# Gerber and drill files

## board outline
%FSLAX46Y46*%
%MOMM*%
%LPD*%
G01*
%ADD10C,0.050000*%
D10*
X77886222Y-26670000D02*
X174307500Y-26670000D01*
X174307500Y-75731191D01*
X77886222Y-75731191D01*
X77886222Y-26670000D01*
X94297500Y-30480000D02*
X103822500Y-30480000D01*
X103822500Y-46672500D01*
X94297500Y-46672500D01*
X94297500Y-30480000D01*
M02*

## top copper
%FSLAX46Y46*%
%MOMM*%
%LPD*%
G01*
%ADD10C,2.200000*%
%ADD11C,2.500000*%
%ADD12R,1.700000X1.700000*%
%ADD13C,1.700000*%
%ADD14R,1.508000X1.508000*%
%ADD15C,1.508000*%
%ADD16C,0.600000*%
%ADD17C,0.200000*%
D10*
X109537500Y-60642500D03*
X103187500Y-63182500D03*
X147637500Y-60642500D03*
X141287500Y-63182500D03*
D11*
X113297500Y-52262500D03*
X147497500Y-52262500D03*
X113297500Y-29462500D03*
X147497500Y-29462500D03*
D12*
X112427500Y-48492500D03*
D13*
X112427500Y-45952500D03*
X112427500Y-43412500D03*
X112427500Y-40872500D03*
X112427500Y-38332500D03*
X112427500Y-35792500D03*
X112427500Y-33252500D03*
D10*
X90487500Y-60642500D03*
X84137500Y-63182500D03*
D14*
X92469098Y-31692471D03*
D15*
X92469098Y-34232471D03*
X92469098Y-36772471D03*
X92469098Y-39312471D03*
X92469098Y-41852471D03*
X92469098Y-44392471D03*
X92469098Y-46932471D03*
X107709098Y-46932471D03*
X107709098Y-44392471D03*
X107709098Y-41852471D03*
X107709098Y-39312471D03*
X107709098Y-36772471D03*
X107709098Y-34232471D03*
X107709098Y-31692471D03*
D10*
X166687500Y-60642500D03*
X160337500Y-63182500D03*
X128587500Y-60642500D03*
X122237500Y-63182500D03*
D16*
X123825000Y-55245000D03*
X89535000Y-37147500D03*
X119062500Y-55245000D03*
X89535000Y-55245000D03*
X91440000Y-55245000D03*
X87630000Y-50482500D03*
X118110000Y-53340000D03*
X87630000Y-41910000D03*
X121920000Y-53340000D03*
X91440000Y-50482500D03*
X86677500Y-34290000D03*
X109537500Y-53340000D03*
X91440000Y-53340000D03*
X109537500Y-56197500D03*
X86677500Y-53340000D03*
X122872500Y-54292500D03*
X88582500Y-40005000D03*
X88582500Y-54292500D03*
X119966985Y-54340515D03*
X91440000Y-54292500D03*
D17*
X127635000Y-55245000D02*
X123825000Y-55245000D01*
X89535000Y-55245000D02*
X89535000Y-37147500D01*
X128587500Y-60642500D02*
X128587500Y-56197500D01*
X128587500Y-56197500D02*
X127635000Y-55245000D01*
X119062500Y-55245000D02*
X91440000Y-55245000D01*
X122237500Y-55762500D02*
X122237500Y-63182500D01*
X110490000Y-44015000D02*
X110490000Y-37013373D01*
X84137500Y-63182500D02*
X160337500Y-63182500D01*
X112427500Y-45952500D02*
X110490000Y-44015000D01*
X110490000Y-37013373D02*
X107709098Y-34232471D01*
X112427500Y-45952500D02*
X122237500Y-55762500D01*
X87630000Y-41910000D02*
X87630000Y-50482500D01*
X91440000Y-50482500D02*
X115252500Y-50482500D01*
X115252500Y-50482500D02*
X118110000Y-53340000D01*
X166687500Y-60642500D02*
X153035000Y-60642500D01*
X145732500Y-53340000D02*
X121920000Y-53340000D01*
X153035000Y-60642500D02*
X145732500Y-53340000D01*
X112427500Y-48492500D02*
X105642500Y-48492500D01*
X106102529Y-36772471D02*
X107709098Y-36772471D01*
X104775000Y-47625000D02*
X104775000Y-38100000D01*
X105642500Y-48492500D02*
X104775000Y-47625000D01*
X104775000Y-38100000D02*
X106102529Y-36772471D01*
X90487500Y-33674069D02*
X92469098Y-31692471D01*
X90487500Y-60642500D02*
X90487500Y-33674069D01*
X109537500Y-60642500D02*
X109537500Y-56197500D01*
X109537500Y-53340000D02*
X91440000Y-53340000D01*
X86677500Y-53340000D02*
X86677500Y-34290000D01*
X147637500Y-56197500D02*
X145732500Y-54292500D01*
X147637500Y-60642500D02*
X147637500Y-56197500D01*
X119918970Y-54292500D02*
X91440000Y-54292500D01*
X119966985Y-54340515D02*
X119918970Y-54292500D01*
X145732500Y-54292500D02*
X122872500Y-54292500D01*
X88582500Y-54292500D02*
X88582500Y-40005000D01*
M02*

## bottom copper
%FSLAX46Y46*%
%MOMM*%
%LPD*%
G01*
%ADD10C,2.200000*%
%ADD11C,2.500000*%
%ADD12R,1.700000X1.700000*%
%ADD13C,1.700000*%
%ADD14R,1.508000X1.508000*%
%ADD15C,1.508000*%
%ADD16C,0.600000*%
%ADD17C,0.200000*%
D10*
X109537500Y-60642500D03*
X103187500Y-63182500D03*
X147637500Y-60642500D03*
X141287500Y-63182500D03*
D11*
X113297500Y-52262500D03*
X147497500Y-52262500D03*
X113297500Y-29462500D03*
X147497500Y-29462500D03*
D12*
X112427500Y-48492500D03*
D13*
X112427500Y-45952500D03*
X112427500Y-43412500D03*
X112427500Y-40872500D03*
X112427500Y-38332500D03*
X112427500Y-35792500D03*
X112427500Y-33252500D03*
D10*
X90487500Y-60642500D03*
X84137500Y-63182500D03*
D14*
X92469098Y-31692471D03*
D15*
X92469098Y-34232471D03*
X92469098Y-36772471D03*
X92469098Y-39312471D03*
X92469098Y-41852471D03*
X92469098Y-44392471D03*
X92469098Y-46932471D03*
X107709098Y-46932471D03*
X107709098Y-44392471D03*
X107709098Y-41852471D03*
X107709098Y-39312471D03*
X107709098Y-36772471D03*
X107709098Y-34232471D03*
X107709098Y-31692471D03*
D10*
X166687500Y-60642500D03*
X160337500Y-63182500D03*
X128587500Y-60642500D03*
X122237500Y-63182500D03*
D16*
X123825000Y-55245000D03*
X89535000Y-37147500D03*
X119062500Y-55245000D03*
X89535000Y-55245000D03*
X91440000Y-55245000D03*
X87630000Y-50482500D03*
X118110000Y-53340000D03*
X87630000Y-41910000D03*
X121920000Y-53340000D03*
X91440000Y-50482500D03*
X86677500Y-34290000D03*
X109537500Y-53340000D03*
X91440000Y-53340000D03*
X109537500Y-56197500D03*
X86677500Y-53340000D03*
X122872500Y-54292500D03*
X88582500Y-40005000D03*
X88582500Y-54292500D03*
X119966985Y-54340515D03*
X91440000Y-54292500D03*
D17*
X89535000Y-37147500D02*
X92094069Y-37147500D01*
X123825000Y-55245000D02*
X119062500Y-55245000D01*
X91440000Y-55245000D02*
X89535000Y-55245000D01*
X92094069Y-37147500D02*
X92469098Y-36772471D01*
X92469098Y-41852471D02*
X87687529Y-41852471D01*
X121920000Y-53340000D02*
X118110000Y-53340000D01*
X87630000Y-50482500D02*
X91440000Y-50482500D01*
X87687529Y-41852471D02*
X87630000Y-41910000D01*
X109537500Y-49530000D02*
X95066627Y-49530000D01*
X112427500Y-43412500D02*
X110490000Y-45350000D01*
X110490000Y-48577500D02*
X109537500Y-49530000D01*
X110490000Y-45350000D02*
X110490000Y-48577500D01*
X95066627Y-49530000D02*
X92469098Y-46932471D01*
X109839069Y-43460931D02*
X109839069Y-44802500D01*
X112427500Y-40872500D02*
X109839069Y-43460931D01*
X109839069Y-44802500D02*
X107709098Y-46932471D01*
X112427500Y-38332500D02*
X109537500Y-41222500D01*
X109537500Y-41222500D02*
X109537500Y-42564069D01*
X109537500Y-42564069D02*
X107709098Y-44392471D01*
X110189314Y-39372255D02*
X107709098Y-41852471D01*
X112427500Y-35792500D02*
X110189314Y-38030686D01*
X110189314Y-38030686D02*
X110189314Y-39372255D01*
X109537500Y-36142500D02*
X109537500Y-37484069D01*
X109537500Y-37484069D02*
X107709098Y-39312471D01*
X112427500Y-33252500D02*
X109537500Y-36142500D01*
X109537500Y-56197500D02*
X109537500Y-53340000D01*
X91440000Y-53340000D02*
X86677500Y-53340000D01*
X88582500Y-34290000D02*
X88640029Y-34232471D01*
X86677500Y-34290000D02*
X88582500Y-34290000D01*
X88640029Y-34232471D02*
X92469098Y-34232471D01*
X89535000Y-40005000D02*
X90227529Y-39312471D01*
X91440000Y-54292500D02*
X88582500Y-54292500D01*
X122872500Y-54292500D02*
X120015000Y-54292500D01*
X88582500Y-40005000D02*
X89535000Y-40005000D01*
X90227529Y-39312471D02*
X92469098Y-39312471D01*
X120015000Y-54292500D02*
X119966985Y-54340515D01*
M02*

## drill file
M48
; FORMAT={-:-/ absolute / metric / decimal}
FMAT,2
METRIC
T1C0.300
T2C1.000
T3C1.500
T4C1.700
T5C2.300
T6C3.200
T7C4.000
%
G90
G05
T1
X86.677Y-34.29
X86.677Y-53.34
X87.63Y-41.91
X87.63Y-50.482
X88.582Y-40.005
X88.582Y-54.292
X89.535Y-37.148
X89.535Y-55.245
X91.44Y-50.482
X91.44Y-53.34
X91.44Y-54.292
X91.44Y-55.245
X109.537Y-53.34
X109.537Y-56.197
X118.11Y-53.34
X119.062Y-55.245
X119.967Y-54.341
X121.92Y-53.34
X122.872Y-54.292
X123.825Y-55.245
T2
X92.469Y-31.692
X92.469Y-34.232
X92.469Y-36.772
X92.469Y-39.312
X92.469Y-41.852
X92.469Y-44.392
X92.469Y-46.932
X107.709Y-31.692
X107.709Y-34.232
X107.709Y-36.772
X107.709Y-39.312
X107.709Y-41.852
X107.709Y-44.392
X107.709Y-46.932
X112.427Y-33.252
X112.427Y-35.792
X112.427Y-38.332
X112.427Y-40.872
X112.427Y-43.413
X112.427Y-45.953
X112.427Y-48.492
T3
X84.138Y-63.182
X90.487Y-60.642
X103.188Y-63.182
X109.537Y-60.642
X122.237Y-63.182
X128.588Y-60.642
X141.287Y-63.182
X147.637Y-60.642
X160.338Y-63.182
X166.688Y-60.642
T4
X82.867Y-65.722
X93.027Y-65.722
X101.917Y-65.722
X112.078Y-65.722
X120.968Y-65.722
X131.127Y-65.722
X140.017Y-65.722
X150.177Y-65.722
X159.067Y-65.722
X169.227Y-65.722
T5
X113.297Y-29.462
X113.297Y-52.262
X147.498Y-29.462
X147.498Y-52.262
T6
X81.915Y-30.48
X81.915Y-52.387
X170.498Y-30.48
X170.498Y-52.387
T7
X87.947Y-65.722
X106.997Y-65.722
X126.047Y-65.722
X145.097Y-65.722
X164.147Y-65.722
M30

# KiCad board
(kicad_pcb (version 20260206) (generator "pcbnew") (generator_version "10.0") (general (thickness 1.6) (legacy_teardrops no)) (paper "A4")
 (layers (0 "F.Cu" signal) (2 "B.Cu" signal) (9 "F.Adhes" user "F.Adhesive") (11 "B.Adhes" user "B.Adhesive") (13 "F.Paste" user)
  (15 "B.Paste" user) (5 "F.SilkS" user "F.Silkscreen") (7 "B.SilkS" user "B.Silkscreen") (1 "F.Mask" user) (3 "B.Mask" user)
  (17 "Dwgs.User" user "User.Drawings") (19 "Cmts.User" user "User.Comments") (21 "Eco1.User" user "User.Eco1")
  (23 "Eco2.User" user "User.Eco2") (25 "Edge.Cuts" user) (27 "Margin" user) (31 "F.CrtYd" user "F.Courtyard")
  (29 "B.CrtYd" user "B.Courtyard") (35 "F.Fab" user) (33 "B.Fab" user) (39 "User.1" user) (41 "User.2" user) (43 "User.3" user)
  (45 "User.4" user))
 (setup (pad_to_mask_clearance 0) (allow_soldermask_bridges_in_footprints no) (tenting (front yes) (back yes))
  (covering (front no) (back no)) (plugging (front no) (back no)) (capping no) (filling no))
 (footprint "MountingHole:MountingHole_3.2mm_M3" (layer "F.Cu") (at 81.915 30.48)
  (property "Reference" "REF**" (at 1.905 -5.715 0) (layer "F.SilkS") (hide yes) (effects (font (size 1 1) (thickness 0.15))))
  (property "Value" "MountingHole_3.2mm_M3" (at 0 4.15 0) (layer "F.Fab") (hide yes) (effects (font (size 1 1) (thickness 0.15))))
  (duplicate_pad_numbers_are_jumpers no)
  (pad "" np_thru_hole circle (at 0 0) (size 3.2 3.2) (drill 3.2) (layers "*.Cu" "*.Mask")))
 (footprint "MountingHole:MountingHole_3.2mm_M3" (layer "F.Cu") (at 170.4975 30.48)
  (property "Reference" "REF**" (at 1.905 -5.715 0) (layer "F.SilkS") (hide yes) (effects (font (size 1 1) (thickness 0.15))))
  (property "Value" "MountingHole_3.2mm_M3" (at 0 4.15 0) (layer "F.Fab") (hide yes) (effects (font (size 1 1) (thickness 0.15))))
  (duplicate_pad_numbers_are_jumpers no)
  (pad "" np_thru_hole circle (at 0 0) (size 3.2 3.2) (drill 3.2) (layers "*.Cu" "*.Mask")))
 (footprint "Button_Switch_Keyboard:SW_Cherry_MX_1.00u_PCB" (layer "F.Cu") (at 109.5375 60.6425)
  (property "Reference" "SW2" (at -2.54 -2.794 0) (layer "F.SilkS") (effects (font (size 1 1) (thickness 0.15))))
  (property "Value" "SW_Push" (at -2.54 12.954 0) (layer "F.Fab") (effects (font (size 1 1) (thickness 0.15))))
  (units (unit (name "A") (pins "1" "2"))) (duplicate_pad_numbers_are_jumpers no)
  (pad "" np_thru_hole circle (at -7.62 5.08) (size 1.7 1.7) (drill 1.7) (layers "*.Cu" "*.Mask"))
  (pad "" np_thru_hole circle (at -2.54 5.08) (size 4 4) (drill 4) (layers "*.Cu" "*.Mask"))
  (pad "" np_thru_hole circle (at 2.54 5.08) (size 1.7 1.7) (drill 1.7) (layers "*.Cu" "*.Mask"))
  (pad "1" thru_hole circle (at 0 0) (size 2.2 2.2) (drill 1.5) (layers "*.Cu" "*.Mask") (remove_unused_layers no)
   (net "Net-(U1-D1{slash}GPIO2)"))
  (pad "2" thru_hole circle (at -6.35 2.54) (size 2.2 2.2) (drill 1.5) (layers "*.Cu" "*.Mask") (remove_unused_layers no) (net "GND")))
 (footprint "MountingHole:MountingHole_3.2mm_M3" (layer "F.Cu") (at 81.915 52.3875)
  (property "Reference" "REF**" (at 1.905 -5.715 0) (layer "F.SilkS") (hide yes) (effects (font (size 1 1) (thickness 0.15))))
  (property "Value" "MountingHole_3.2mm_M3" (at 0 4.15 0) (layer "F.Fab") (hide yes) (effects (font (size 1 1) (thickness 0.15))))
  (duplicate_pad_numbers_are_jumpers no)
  (pad "" np_thru_hole circle (at 0 0) (size 3.2 3.2) (drill 3.2) (layers "*.Cu" "*.Mask")))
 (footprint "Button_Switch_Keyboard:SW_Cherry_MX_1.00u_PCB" (layer "F.Cu") (at 147.6375 60.6425)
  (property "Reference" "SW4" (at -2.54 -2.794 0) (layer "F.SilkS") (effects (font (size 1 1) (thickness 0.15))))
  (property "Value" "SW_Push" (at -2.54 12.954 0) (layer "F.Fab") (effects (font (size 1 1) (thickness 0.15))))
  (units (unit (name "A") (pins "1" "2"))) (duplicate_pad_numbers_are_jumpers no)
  (pad "" np_thru_hole circle (at -7.62 5.08) (size 1.7 1.7) (drill 1.7) (layers "*.Cu" "*.Mask"))
  (pad "" np_thru_hole circle (at -2.54 5.08) (size 4 4) (drill 4) (layers "*.Cu" "*.Mask"))
  (pad "" np_thru_hole circle (at 2.54 5.08) (size 1.7 1.7) (drill 1.7) (layers "*.Cu" "*.Mask"))
  (pad "1" thru_hole circle (at 0 0) (size 2.2 2.2) (drill 1.5) (layers "*.Cu" "*.Mask") (remove_unused_layers no)
   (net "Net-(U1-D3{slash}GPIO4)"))
  (pad "2" thru_hole circle (at -6.35 2.54) (size 2.2 2.2) (drill 1.5) (layers "*.Cu" "*.Mask") (remove_unused_layers no) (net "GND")))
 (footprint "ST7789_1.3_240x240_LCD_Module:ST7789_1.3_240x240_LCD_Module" (layer "F.Cu") (at 149.9975 54.7625 90)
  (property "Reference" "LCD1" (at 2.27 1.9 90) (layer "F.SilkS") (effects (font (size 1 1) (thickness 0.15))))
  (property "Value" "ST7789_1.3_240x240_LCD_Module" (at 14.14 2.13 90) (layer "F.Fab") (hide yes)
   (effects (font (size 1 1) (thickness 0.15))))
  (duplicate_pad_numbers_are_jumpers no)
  (pad "" np_thru_hole circle (at 2.5 -36.7 90) (size 2.5 2.5) (drill 2.3) (layers "*.Cu" "*.Mask"))
  (pad "" np_thru_hole circle (at 2.5 -2.5 90) (size 2.5 2.5) (drill 2.3) (layers "*.Cu" "*.Mask"))
  (pad "" np_thru_hole circle (at 25.3 -36.7 90) (size 2.5 2.5) (drill 2.3) (layers "*.Cu" "*.Mask"))
  (pad "" np_thru_hole circle (at 25.3 -2.5 90) (size 2.5 2.5) (drill 2.3) (layers "*.Cu" "*.Mask"))
  (pad "1" thru_hole rect (at 6.27 -37.57 90) (size 1.7 1.7) (drill 1) (layers "*.Cu" "*.Mask") (remove_unused_layers no)
   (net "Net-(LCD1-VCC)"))
  (pad "2" thru_hole circle (at 8.81 -37.57 90) (size 1.7 1.7) (drill 1) (layers "*.Cu" "*.Mask") (remove_unused_layers no) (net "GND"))
  (pad "3" thru_hole circle (at 11.35 -37.57 90) (size 1.7 1.7) (drill 1) (layers "*.Cu" "*.Mask") (remove_unused_layers no)
   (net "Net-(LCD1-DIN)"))
  (pad "4" thru_hole circle (at 13.89 -37.57 90) (size 1.7 1.7) (drill 1) (layers "*.Cu" "*.Mask") (remove_unused_layers no)
   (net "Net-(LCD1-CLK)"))
  (pad "5" thru_hole circle (at 16.43 -37.57 90) (size 1.7 1.7) (drill 1) (layers "*.Cu" "*.Mask") (remove_unused_layers no)
   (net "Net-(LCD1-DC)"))
  (pad "6" thru_hole circle (at 18.97 -37.57 90) (size 1.7 1.7) (drill 1) (layers "*.Cu" "*.Mask") (remove_unused_layers no)
   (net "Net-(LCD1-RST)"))
  (pad "7" thru_hole circle (at 21.51 -37.57 90) (size 1.7 1.7) (drill 1) (layers "*.Cu" "*.Mask") (remove_unused_layers no)
   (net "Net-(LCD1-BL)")))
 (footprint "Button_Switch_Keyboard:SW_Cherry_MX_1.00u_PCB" (layer "F.Cu") (at 90.4875 60.6425)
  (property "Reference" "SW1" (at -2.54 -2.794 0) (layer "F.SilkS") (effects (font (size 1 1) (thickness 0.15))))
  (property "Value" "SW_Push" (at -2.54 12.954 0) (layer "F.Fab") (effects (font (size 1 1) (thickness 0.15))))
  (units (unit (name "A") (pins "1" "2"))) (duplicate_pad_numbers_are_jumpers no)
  (pad "" np_thru_hole circle (at -7.62 5.08) (size 1.7 1.7) (drill 1.7) (layers "*.Cu" "*.Mask"))
  (pad "" np_thru_hole circle (at -2.54 5.08) (size 4 4) (drill 4) (layers "*.Cu" "*.Mask"))
  (pad "" np_thru_hole circle (at 2.54 5.08) (size 1.7 1.7) (drill 1.7) (layers "*.Cu" "*.Mask"))
  (pad "1" thru_hole circle (at 0 0) (size 2.2 2.2) (drill 1.5) (layers "*.Cu" "*.Mask") (remove_unused_layers no)
   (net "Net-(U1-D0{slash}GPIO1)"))
  (pad "2" thru_hole circle (at -6.35 2.54) (size 2.2 2.2) (drill 1.5) (layers "*.Cu" "*.Mask") (remove_unused_layers no) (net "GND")))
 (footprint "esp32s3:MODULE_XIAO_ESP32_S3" (layer "F.Cu") (at 100.089098 39.248971)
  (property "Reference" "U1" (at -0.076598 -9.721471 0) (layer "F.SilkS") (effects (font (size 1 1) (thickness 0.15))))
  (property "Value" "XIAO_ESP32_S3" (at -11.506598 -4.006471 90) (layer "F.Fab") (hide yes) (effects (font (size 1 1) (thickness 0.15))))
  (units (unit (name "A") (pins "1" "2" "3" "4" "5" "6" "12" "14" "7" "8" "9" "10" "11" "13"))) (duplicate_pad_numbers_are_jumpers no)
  (pad "1" thru_hole rect (at -7.62 -7.5565) (size 1.508 1.508) (drill 1) (layers "*.Cu" "*.Mask") (remove_unused_layers no)
   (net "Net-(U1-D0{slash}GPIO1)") (solder_mask_margin 0.102))
  (pad "2" thru_hole circle (at -7.62 -5.0165) (size 1.508 1.508) (drill 1) (layers "*.Cu" "*.Mask") (remove_unused_layers no)
   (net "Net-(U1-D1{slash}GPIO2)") (solder_mask_margin 0.102))
  (pad "3" thru_hole circle (at -7.62 -2.4765) (size 1.508 1.508) (drill 1) (layers "*.Cu" "*.Mask") (remove_unused_layers no)
   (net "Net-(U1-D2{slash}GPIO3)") (solder_mask_margin 0.102))
  (pad "4" thru_hole circle (at -7.62 0.0635) (size 1.508 1.508) (drill 1) (layers "*.Cu" "*.Mask") (remove_unused_layers no)
   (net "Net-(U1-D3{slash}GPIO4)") (solder_mask_margin 0.102))
  (pad "5" thru_hole circle (at -7.62 2.6035) (size 1.508 1.508) (drill 1) (layers "*.Cu" "*.Mask") (remove_unused_layers no)
   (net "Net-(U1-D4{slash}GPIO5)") (solder_mask_margin 0.102))
  (pad "6" thru_hole circle (at -7.62 5.1435) (size 1.508 1.508) (drill 1) (layers "*.Cu" "*.Mask") (remove_unused_layers no)
   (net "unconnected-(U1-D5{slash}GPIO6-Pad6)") (solder_mask_margin 0.102))
  (pad "7" thru_hole circle (at -7.62 7.6835) (size 1.508 1.508) (drill 1) (layers "*.Cu" "*.Mask") (remove_unused_layers no)
   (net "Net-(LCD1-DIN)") (solder_mask_margin 0.102))
  (pad "8" thru_hole circle (at 7.62 7.6835) (size 1.508 1.508) (drill 1) (layers "*.Cu" "*.Mask") (remove_unused_layers no)
   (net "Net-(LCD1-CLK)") (solder_mask_margin 0.102))
  (pad "9" thru_hole circle (at 7.62 5.1435) (size 1.508 1.508) (drill 1) (layers "*.Cu" "*.Mask") (remove_unused_layers no)
   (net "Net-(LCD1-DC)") (solder_mask_margin 0.102))
  (pad "10" thru_hole circle (at 7.62 2.6035) (size 1.508 1.508) (drill 1) (layers "*.Cu" "*.Mask") (remove_unused_layers no)
   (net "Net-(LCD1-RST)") (solder_mask_margin 0.102))
  (pad "11" thru_hole circle (at 7.62 0.0635) (size 1.508 1.508) (drill 1) (layers "*.Cu" "*.Mask") (remove_unused_layers no)
   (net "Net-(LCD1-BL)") (solder_mask_margin 0.102))
  (pad "12" thru_hole circle (at 7.62 -2.4765) (size 1.508 1.508) (drill 1) (layers "*.Cu" "*.Mask") (remove_unused_layers no)
   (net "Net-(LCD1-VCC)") (solder_mask_margin 0.102))
  (pad "13" thru_hole circle (at 7.62 -5.0165) (size 1.508 1.508) (drill 1) (layers "*.Cu" "*.Mask") (remove_unused_layers no) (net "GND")
   (solder_mask_margin 0.102))
  (pad "14" thru_hole circle (at 7.62 -7.5565) (size 1.508 1.508) (drill 1) (layers "*.Cu" "*.Mask") (remove_unused_layers no)
   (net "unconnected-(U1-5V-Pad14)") (solder_mask_margin 0.102)))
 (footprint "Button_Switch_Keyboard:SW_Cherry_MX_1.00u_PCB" (layer "F.Cu") (at 166.6875 60.6425)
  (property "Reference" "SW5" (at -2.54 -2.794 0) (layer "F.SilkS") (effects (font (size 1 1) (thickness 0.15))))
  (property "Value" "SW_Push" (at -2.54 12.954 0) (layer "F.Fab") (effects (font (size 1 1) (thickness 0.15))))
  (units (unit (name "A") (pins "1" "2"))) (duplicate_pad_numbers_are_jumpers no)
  (pad "" np_thru_hole circle (at -7.62 5.08) (size 1.7 1.7) (drill 1.7) (layers "*.Cu" "*.Mask"))
  (pad "" np_thru_hole circle (at -2.54 5.08) (size 4 4) (drill 4) (layers "*.Cu" "*.Mask"))
  (pad "" np_thru_hole circle (at 2.54 5.08) (size 1.7 1.7) (drill 1.7) (layers "*.Cu" "*.Mask"))
  (pad "1" thru_hole circle (at 0 0) (size 2.2 2.2) (drill 1.5) (layers "*.Cu" "*.Mask") (remove_unused_layers no)
   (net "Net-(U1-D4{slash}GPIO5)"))
  (pad "2" thru_hole circle (at -6.35 2.54) (size 2.2 2.2) (drill 1.5) (layers "*.Cu" "*.Mask") (remove_unused_layers no) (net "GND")))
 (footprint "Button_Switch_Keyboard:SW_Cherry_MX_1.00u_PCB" (layer "F.Cu") (at 128.5875 60.6425)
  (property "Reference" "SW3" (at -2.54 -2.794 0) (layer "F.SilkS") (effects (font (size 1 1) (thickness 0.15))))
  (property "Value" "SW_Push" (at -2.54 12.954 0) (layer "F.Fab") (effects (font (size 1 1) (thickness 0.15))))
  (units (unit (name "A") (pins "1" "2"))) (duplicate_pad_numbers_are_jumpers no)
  (pad "" np_thru_hole circle (at -7.62 5.08) (size 1.7 1.7) (drill 1.7) (layers "*.Cu" "*.Mask"))
  (pad "" np_thru_hole circle (at -2.54 5.08) (size 4 4) (drill 4) (layers "*.Cu" "*.Mask"))
  (pad "" np_thru_hole circle (at 2.54 5.08) (size 1.7 1.7) (drill 1.7) (layers "*.Cu" "*.Mask"))
  (pad "1" thru_hole circle (at 0 0) (size 2.2 2.2) (drill 1.5) (layers "*.Cu" "*.Mask") (remove_unused_layers no)
   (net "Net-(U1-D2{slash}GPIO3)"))
  (pad "2" thru_hole circle (at -6.35 2.54) (size 2.2 2.2) (drill 1.5) (layers "*.Cu" "*.Mask") (remove_unused_layers no) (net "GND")))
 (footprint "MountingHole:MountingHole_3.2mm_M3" (layer "F.Cu") (at 170.4975 52.3875)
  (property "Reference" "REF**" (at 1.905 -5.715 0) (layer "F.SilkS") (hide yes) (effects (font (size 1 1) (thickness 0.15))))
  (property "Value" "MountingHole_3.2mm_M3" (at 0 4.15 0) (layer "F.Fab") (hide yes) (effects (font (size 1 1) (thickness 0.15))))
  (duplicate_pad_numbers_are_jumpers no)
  (pad "" np_thru_hole circle (at 0 0) (size 3.2 3.2) (drill 3.2) (layers "*.Cu" "*.Mask")))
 (gr_rect (start 77.886222 26.67) (end 174.3075 75.731191) (stroke (width 0.05) (type default)) (fill no) (layer "Edge.Cuts"))
 (gr_rect (start 94.2975 30.48) (end 103.8225 46.6725) (stroke (width 0.05) (type default)) (fill no) (layer "Edge.Cuts"))
 (segment (start 127.635 55.245) (end 123.825 55.245) (width 0.2) (layer "F.Cu") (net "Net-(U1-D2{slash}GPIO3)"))
 (segment (start 89.535 55.245) (end 89.535 37.1475) (width 0.2) (layer "F.Cu") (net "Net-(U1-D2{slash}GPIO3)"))
 (segment (start 128.5875 60.6425) (end 128.5875 56.1975) (width 0.2) (layer "F.Cu") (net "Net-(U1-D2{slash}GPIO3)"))
 (segment (start 128.5875 56.1975) (end 127.635 55.245) (width 0.2) (layer "F.Cu") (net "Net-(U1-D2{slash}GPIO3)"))
 (segment (start 119.0625 55.245) (end 91.44 55.245) (width 0.2) (layer "F.Cu") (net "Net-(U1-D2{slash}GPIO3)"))
 (via (at 123.825 55.245) (size 0.6) (drill 0.3) (layers "F.Cu" "B.Cu") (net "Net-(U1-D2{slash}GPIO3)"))
 (via (at 89.535 37.1475) (size 0.6) (drill 0.3) (layers "F.Cu" "B.Cu") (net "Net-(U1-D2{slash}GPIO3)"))
 (via (at 119.0625 55.245) (size 0.6) (drill 0.3) (layers "F.Cu" "B.Cu") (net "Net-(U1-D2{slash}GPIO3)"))
 (via (at 89.535 55.245) (size 0.6) (drill 0.3) (layers "F.Cu" "B.Cu") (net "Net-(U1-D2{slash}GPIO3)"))
 (via (at 91.44 55.245) (size 0.6) (drill 0.3) (layers "F.Cu" "B.Cu") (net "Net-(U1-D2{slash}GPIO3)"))
 (segment (start 89.535 37.1475) (end 92.094069 37.1475) (width 0.2) (layer "B.Cu") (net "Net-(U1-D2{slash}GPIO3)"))
 (segment (start 123.825 55.245) (end 119.0625 55.245) (width 0.2) (layer "B.Cu") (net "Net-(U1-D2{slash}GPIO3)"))
 (segment (start 91.44 55.245) (end 89.535 55.245) (width 0.2) (layer "B.Cu") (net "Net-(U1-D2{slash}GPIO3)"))
 (segment (start 92.094069 37.1475) (end 92.469098 36.772471) (width 0.2) (layer "B.Cu") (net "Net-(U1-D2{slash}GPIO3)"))
 (segment (start 122.2375 55.7625) (end 122.2375 63.1825) (width 0.2) (layer "F.Cu") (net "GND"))
 (segment (start 110.49 44.015) (end 110.49 37.013373) (width 0.2) (layer "F.Cu") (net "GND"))
 (segment (start 84.1375 63.1825) (end 160.3375 63.1825) (width 0.2) (layer "F.Cu") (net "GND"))
 (segment (start 112.4275 45.9525) (end 110.49 44.015) (width 0.2) (layer "F.Cu") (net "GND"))
 (segment (start 110.49 37.013373) (end 107.709098 34.232471) (width 0.2) (layer "F.Cu") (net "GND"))
 (segment (start 112.4275 45.9525) (end 122.2375 55.7625) (width 0.2) (layer "F.Cu") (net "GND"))
 (segment (start 87.63 41.91) (end 87.63 50.4825) (width 0.2) (layer "F.Cu") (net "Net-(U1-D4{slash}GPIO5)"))
 (segment (start 91.44 50.4825) (end 115.2525 50.4825) (width 0.2) (layer "F.Cu") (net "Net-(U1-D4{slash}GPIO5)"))
 (segment (start 115.2525 50.4825) (end 118.11 53.34) (width 0.2) (layer "F.Cu") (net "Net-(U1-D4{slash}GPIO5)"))
 (segment (start 166.6875 60.6425) (end 153.035 60.6425) (width 0.2) (layer "F.Cu") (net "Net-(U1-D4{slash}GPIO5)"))
 (segment (start 145.7325 53.34) (end 121.92 53.34) (width 0.2) (layer "F.Cu") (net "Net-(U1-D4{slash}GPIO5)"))
 (segment (start 153.035 60.6425) (end 145.7325 53.34) (width 0.2) (layer "F.Cu") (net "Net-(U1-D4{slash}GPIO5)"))
 (via (at 87.63 50.4825) (size 0.6) (drill 0.3) (layers "F.Cu" "B.Cu") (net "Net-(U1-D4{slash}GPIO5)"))
 (via (at 118.11 53.34) (size 0.6) (drill 0.3) (layers "F.Cu" "B.Cu") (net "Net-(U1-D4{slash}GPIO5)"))
 (via (at 87.63 41.91) (size 0.6) (drill 0.3) (layers "F.Cu" "B.Cu") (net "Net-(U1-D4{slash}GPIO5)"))
 (via (at 121.92 53.34) (size 0.6) (drill 0.3) (layers "F.Cu" "B.Cu") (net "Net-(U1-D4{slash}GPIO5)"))
 (via (at 91.44 50.4825) (size 0.6) (drill 0.3) (layers "F.Cu" "B.Cu") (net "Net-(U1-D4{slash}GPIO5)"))
 (segment (start 92.469098 41.852471) (end 87.687529 41.852471) (width 0.2) (layer "B.Cu") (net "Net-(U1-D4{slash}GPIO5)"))
 (segment (start 121.92 53.34) (end 118.11 53.34) (width 0.2) (layer "B.Cu") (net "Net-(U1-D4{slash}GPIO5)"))
 (segment (start 87.63 50.4825) (end 91.44 50.4825) (width 0.2) (layer "B.Cu") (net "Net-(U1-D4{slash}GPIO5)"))
 (segment (start 87.687529 41.852471) (end 87.63 41.91) (width 0.2) (layer "B.Cu") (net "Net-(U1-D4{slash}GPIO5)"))
 (segment (start 112.4275 48.4925) (end 105.6425 48.4925) (width 0.2) (layer "F.Cu") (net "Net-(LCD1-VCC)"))
 (segment (start 106.102529 36.772471) (end 107.709098 36.772471) (width 0.2) (layer "F.Cu") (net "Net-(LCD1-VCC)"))
 (segment (start 104.775 47.625) (end 104.775 38.1) (width 0.2) (layer "F.Cu") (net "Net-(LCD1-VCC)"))
 (segment (start 105.6425 48.4925) (end 104.775 47.625) (width 0.2) (layer "F.Cu") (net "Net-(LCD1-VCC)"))
 (segment (start 104.775 38.1) (end 106.102529 36.772471) (width 0.2) (layer "F.Cu") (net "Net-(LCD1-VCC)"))
 (segment (start 109.5375 49.53) (end 95.066627 49.53) (width 0.2) (layer "B.Cu") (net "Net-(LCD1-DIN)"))
 (segment (start 112.4275 43.4125) (end 110.49 45.35) (width 0.2) (layer "B.Cu") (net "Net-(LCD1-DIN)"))
 (segment (start 110.49 48.5775) (end 109.5375 49.53) (width 0.2) (layer "B.Cu") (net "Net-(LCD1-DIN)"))
 (segment (start 110.49 45.35) (end 110.49 48.5775) (width 0.2) (layer "B.Cu") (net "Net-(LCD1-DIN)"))
 (segment (start 95.066627 49.53) (end 92.469098 46.932471) (width 0.2) (layer "B.Cu") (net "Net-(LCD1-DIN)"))
 (segment (start 109.839069 43.460931) (end 109.839069 44.8025) (width 0.2) (layer "B.Cu") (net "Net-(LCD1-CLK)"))
 (segment (start 112.4275 40.8725) (end 109.839069 43.460931) (width 0.2) (layer "B.Cu") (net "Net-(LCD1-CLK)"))
 (segment (start 109.839069 44.8025) (end 107.709098 46.932471) (width 0.2) (layer "B.Cu") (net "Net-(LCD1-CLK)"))
 (segment (start 112.4275 38.3325) (end 109.5375 41.2225) (width 0.2) (layer "B.Cu") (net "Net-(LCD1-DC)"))
 (segment (start 109.5375 41.2225) (end 109.5375 42.564069) (width 0.2) (layer "B.Cu") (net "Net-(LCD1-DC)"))
 (segment (start 109.5375 42.564069) (end 107.709098 44.392471) (width 0.2) (layer "B.Cu") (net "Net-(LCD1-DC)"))
 (segment (start 110.189314 39.372255) (end 107.709098 41.852471) (width 0.2) (layer "B.Cu") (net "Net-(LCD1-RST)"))
 (segment (start 112.4275 35.7925) (end 110.189314 38.030686) (width 0.2) (layer "B.Cu") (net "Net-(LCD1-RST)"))
 (segment (start 110.189314 38.030686) (end 110.189314 39.372255) (width 0.2) (layer "B.Cu") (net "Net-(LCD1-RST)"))
 (segment (start 109.5375 36.1425) (end 109.5375 37.484069) (width 0.2) (layer "B.Cu") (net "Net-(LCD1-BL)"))
 (segment (start 109.5375 37.484069) (end 107.709098 39.312471) (width 0.2) (layer "B.Cu") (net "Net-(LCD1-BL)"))
 (segment (start 112.4275 33.2525) (end 109.5375 36.1425) (width 0.2) (layer "B.Cu") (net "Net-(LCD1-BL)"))
 (segment (start 90.4875 33.674069) (end 92.469098 31.692471) (width 0.2) (layer "F.Cu") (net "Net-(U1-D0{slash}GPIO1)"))
 (segment (start 90.4875 60.6425) (end 90.4875 33.674069) (width 0.2) (layer "F.Cu") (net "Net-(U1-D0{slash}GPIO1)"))
 (segment (start 109.5375 60.6425) (end 109.5375 56.1975) (width 0.2) (layer "F.Cu") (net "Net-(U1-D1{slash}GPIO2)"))
 (segment (start 109.5375 53.34) (end 91.44 53.34) (width 0.2) (layer "F.Cu") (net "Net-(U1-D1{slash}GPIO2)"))
 (segment (start 86.6775 53.34) (end 86.6775 34.29) (width 0.2) (layer "F.Cu") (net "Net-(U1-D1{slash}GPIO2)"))
 (via (at 86.6775 34.29) (size 0.6) (drill 0.3) (layers "F.Cu" "B.Cu") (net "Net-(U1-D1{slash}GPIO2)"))
 (via (at 109.5375 53.34) (size 0.6) (drill 0.3) (layers "F.Cu" "B.Cu") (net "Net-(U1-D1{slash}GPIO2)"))
 (via (at 91.44 53.34) (size 0.6) (drill 0.3) (layers "F.Cu" "B.Cu") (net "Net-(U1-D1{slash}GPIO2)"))
 (via (at 109.5375 56.1975) (size 0.6) (drill 0.3) (layers "F.Cu" "B.Cu") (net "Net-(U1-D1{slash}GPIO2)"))
 (via (at 86.6775 53.34) (size 0.6) (drill 0.3) (layers "F.Cu" "B.Cu") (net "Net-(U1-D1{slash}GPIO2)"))
 (segment (start 109.5375 56.1975) (end 109.5375 53.34) (width 0.2) (layer "B.Cu") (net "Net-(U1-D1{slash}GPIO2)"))
 (segment (start 91.44 53.34) (end 86.6775 53.34) (width 0.2) (layer "B.Cu") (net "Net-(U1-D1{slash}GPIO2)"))
 (segment (start 88.5825 34.29) (end 88.640029 34.232471) (width 0.2) (layer "B.Cu") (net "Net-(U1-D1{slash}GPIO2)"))
 (segment (start 86.6775 34.29) (end 88.5825 34.29) (width 0.2) (layer "B.Cu") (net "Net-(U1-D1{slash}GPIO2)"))
 (segment (start 88.640029 34.232471) (end 92.469098 34.232471) (width 0.2) (layer "B.Cu") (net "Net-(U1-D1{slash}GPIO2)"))
 (segment (start 147.6375 56.1975) (end 145.7325 54.2925) (width 0.2) (layer "F.Cu") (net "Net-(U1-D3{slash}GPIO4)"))
 (segment (start 147.6375 60.6425) (end 147.6375 56.1975) (width 0.2) (layer "F.Cu") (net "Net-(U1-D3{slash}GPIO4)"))
 (segment (start 119.91897 54.2925) (end 91.44 54.2925) (width 0.2) (layer "F.Cu") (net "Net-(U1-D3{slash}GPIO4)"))
 (segment (start 119.966985 54.340515) (end 119.91897 54.2925) (width 0.2) (layer "F.Cu") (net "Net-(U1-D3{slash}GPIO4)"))
 (segment (start 145.7325 54.2925) (end 122.8725 54.2925) (width 0.2) (layer "F.Cu") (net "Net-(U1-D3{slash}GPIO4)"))
 (segment (start 88.5825 54.2925) (end 88.5825 40.005) (width 0.2) (layer "F.Cu") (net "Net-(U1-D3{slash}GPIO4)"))
 (via (at 122.8725 54.2925) (size 0.6) (drill 0.3) (layers "F.Cu" "B.Cu") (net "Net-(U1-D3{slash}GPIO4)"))
 (via (at 88.5825 40.005) (size 0.6) (drill 0.3) (layers "F.Cu" "B.Cu") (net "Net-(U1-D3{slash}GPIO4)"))
 (via (at 88.5825 54.2925) (size 0.6) (drill 0.3) (layers "F.Cu" "B.Cu") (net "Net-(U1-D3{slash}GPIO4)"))
 (via (at 119.966985 54.340515) (size 0.6) (drill 0.3) (layers "F.Cu" "B.Cu") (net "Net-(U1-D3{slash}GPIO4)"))
 (via (at 91.44 54.2925) (size 0.6) (drill 0.3) (layers "F.Cu" "B.Cu") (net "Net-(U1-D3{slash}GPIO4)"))
 (segment (start 89.535 40.005) (end 90.227529 39.312471) (width 0.2) (layer "B.Cu") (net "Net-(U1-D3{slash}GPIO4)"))
 (segment (start 91.44 54.2925) (end 88.5825 54.2925) (width 0.2) (layer "B.Cu") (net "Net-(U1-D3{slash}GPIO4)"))
 (segment (start 122.8725 54.2925) (end 120.015 54.2925) (width 0.2) (layer "B.Cu") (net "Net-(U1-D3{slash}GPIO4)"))
 (segment (start 88.5825 40.005) (end 89.535 40.005) (width 0.2) (layer "B.Cu") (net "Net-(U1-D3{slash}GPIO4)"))
 (segment (start 90.227529 39.312471) (end 92.469098 39.312471) (width 0.2) (layer "B.Cu") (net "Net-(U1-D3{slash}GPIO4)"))
 (segment (start 120.015 54.2925) (end 119.966985 54.340515) (width 0.2) (layer "B.Cu") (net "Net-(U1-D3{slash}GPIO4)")))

